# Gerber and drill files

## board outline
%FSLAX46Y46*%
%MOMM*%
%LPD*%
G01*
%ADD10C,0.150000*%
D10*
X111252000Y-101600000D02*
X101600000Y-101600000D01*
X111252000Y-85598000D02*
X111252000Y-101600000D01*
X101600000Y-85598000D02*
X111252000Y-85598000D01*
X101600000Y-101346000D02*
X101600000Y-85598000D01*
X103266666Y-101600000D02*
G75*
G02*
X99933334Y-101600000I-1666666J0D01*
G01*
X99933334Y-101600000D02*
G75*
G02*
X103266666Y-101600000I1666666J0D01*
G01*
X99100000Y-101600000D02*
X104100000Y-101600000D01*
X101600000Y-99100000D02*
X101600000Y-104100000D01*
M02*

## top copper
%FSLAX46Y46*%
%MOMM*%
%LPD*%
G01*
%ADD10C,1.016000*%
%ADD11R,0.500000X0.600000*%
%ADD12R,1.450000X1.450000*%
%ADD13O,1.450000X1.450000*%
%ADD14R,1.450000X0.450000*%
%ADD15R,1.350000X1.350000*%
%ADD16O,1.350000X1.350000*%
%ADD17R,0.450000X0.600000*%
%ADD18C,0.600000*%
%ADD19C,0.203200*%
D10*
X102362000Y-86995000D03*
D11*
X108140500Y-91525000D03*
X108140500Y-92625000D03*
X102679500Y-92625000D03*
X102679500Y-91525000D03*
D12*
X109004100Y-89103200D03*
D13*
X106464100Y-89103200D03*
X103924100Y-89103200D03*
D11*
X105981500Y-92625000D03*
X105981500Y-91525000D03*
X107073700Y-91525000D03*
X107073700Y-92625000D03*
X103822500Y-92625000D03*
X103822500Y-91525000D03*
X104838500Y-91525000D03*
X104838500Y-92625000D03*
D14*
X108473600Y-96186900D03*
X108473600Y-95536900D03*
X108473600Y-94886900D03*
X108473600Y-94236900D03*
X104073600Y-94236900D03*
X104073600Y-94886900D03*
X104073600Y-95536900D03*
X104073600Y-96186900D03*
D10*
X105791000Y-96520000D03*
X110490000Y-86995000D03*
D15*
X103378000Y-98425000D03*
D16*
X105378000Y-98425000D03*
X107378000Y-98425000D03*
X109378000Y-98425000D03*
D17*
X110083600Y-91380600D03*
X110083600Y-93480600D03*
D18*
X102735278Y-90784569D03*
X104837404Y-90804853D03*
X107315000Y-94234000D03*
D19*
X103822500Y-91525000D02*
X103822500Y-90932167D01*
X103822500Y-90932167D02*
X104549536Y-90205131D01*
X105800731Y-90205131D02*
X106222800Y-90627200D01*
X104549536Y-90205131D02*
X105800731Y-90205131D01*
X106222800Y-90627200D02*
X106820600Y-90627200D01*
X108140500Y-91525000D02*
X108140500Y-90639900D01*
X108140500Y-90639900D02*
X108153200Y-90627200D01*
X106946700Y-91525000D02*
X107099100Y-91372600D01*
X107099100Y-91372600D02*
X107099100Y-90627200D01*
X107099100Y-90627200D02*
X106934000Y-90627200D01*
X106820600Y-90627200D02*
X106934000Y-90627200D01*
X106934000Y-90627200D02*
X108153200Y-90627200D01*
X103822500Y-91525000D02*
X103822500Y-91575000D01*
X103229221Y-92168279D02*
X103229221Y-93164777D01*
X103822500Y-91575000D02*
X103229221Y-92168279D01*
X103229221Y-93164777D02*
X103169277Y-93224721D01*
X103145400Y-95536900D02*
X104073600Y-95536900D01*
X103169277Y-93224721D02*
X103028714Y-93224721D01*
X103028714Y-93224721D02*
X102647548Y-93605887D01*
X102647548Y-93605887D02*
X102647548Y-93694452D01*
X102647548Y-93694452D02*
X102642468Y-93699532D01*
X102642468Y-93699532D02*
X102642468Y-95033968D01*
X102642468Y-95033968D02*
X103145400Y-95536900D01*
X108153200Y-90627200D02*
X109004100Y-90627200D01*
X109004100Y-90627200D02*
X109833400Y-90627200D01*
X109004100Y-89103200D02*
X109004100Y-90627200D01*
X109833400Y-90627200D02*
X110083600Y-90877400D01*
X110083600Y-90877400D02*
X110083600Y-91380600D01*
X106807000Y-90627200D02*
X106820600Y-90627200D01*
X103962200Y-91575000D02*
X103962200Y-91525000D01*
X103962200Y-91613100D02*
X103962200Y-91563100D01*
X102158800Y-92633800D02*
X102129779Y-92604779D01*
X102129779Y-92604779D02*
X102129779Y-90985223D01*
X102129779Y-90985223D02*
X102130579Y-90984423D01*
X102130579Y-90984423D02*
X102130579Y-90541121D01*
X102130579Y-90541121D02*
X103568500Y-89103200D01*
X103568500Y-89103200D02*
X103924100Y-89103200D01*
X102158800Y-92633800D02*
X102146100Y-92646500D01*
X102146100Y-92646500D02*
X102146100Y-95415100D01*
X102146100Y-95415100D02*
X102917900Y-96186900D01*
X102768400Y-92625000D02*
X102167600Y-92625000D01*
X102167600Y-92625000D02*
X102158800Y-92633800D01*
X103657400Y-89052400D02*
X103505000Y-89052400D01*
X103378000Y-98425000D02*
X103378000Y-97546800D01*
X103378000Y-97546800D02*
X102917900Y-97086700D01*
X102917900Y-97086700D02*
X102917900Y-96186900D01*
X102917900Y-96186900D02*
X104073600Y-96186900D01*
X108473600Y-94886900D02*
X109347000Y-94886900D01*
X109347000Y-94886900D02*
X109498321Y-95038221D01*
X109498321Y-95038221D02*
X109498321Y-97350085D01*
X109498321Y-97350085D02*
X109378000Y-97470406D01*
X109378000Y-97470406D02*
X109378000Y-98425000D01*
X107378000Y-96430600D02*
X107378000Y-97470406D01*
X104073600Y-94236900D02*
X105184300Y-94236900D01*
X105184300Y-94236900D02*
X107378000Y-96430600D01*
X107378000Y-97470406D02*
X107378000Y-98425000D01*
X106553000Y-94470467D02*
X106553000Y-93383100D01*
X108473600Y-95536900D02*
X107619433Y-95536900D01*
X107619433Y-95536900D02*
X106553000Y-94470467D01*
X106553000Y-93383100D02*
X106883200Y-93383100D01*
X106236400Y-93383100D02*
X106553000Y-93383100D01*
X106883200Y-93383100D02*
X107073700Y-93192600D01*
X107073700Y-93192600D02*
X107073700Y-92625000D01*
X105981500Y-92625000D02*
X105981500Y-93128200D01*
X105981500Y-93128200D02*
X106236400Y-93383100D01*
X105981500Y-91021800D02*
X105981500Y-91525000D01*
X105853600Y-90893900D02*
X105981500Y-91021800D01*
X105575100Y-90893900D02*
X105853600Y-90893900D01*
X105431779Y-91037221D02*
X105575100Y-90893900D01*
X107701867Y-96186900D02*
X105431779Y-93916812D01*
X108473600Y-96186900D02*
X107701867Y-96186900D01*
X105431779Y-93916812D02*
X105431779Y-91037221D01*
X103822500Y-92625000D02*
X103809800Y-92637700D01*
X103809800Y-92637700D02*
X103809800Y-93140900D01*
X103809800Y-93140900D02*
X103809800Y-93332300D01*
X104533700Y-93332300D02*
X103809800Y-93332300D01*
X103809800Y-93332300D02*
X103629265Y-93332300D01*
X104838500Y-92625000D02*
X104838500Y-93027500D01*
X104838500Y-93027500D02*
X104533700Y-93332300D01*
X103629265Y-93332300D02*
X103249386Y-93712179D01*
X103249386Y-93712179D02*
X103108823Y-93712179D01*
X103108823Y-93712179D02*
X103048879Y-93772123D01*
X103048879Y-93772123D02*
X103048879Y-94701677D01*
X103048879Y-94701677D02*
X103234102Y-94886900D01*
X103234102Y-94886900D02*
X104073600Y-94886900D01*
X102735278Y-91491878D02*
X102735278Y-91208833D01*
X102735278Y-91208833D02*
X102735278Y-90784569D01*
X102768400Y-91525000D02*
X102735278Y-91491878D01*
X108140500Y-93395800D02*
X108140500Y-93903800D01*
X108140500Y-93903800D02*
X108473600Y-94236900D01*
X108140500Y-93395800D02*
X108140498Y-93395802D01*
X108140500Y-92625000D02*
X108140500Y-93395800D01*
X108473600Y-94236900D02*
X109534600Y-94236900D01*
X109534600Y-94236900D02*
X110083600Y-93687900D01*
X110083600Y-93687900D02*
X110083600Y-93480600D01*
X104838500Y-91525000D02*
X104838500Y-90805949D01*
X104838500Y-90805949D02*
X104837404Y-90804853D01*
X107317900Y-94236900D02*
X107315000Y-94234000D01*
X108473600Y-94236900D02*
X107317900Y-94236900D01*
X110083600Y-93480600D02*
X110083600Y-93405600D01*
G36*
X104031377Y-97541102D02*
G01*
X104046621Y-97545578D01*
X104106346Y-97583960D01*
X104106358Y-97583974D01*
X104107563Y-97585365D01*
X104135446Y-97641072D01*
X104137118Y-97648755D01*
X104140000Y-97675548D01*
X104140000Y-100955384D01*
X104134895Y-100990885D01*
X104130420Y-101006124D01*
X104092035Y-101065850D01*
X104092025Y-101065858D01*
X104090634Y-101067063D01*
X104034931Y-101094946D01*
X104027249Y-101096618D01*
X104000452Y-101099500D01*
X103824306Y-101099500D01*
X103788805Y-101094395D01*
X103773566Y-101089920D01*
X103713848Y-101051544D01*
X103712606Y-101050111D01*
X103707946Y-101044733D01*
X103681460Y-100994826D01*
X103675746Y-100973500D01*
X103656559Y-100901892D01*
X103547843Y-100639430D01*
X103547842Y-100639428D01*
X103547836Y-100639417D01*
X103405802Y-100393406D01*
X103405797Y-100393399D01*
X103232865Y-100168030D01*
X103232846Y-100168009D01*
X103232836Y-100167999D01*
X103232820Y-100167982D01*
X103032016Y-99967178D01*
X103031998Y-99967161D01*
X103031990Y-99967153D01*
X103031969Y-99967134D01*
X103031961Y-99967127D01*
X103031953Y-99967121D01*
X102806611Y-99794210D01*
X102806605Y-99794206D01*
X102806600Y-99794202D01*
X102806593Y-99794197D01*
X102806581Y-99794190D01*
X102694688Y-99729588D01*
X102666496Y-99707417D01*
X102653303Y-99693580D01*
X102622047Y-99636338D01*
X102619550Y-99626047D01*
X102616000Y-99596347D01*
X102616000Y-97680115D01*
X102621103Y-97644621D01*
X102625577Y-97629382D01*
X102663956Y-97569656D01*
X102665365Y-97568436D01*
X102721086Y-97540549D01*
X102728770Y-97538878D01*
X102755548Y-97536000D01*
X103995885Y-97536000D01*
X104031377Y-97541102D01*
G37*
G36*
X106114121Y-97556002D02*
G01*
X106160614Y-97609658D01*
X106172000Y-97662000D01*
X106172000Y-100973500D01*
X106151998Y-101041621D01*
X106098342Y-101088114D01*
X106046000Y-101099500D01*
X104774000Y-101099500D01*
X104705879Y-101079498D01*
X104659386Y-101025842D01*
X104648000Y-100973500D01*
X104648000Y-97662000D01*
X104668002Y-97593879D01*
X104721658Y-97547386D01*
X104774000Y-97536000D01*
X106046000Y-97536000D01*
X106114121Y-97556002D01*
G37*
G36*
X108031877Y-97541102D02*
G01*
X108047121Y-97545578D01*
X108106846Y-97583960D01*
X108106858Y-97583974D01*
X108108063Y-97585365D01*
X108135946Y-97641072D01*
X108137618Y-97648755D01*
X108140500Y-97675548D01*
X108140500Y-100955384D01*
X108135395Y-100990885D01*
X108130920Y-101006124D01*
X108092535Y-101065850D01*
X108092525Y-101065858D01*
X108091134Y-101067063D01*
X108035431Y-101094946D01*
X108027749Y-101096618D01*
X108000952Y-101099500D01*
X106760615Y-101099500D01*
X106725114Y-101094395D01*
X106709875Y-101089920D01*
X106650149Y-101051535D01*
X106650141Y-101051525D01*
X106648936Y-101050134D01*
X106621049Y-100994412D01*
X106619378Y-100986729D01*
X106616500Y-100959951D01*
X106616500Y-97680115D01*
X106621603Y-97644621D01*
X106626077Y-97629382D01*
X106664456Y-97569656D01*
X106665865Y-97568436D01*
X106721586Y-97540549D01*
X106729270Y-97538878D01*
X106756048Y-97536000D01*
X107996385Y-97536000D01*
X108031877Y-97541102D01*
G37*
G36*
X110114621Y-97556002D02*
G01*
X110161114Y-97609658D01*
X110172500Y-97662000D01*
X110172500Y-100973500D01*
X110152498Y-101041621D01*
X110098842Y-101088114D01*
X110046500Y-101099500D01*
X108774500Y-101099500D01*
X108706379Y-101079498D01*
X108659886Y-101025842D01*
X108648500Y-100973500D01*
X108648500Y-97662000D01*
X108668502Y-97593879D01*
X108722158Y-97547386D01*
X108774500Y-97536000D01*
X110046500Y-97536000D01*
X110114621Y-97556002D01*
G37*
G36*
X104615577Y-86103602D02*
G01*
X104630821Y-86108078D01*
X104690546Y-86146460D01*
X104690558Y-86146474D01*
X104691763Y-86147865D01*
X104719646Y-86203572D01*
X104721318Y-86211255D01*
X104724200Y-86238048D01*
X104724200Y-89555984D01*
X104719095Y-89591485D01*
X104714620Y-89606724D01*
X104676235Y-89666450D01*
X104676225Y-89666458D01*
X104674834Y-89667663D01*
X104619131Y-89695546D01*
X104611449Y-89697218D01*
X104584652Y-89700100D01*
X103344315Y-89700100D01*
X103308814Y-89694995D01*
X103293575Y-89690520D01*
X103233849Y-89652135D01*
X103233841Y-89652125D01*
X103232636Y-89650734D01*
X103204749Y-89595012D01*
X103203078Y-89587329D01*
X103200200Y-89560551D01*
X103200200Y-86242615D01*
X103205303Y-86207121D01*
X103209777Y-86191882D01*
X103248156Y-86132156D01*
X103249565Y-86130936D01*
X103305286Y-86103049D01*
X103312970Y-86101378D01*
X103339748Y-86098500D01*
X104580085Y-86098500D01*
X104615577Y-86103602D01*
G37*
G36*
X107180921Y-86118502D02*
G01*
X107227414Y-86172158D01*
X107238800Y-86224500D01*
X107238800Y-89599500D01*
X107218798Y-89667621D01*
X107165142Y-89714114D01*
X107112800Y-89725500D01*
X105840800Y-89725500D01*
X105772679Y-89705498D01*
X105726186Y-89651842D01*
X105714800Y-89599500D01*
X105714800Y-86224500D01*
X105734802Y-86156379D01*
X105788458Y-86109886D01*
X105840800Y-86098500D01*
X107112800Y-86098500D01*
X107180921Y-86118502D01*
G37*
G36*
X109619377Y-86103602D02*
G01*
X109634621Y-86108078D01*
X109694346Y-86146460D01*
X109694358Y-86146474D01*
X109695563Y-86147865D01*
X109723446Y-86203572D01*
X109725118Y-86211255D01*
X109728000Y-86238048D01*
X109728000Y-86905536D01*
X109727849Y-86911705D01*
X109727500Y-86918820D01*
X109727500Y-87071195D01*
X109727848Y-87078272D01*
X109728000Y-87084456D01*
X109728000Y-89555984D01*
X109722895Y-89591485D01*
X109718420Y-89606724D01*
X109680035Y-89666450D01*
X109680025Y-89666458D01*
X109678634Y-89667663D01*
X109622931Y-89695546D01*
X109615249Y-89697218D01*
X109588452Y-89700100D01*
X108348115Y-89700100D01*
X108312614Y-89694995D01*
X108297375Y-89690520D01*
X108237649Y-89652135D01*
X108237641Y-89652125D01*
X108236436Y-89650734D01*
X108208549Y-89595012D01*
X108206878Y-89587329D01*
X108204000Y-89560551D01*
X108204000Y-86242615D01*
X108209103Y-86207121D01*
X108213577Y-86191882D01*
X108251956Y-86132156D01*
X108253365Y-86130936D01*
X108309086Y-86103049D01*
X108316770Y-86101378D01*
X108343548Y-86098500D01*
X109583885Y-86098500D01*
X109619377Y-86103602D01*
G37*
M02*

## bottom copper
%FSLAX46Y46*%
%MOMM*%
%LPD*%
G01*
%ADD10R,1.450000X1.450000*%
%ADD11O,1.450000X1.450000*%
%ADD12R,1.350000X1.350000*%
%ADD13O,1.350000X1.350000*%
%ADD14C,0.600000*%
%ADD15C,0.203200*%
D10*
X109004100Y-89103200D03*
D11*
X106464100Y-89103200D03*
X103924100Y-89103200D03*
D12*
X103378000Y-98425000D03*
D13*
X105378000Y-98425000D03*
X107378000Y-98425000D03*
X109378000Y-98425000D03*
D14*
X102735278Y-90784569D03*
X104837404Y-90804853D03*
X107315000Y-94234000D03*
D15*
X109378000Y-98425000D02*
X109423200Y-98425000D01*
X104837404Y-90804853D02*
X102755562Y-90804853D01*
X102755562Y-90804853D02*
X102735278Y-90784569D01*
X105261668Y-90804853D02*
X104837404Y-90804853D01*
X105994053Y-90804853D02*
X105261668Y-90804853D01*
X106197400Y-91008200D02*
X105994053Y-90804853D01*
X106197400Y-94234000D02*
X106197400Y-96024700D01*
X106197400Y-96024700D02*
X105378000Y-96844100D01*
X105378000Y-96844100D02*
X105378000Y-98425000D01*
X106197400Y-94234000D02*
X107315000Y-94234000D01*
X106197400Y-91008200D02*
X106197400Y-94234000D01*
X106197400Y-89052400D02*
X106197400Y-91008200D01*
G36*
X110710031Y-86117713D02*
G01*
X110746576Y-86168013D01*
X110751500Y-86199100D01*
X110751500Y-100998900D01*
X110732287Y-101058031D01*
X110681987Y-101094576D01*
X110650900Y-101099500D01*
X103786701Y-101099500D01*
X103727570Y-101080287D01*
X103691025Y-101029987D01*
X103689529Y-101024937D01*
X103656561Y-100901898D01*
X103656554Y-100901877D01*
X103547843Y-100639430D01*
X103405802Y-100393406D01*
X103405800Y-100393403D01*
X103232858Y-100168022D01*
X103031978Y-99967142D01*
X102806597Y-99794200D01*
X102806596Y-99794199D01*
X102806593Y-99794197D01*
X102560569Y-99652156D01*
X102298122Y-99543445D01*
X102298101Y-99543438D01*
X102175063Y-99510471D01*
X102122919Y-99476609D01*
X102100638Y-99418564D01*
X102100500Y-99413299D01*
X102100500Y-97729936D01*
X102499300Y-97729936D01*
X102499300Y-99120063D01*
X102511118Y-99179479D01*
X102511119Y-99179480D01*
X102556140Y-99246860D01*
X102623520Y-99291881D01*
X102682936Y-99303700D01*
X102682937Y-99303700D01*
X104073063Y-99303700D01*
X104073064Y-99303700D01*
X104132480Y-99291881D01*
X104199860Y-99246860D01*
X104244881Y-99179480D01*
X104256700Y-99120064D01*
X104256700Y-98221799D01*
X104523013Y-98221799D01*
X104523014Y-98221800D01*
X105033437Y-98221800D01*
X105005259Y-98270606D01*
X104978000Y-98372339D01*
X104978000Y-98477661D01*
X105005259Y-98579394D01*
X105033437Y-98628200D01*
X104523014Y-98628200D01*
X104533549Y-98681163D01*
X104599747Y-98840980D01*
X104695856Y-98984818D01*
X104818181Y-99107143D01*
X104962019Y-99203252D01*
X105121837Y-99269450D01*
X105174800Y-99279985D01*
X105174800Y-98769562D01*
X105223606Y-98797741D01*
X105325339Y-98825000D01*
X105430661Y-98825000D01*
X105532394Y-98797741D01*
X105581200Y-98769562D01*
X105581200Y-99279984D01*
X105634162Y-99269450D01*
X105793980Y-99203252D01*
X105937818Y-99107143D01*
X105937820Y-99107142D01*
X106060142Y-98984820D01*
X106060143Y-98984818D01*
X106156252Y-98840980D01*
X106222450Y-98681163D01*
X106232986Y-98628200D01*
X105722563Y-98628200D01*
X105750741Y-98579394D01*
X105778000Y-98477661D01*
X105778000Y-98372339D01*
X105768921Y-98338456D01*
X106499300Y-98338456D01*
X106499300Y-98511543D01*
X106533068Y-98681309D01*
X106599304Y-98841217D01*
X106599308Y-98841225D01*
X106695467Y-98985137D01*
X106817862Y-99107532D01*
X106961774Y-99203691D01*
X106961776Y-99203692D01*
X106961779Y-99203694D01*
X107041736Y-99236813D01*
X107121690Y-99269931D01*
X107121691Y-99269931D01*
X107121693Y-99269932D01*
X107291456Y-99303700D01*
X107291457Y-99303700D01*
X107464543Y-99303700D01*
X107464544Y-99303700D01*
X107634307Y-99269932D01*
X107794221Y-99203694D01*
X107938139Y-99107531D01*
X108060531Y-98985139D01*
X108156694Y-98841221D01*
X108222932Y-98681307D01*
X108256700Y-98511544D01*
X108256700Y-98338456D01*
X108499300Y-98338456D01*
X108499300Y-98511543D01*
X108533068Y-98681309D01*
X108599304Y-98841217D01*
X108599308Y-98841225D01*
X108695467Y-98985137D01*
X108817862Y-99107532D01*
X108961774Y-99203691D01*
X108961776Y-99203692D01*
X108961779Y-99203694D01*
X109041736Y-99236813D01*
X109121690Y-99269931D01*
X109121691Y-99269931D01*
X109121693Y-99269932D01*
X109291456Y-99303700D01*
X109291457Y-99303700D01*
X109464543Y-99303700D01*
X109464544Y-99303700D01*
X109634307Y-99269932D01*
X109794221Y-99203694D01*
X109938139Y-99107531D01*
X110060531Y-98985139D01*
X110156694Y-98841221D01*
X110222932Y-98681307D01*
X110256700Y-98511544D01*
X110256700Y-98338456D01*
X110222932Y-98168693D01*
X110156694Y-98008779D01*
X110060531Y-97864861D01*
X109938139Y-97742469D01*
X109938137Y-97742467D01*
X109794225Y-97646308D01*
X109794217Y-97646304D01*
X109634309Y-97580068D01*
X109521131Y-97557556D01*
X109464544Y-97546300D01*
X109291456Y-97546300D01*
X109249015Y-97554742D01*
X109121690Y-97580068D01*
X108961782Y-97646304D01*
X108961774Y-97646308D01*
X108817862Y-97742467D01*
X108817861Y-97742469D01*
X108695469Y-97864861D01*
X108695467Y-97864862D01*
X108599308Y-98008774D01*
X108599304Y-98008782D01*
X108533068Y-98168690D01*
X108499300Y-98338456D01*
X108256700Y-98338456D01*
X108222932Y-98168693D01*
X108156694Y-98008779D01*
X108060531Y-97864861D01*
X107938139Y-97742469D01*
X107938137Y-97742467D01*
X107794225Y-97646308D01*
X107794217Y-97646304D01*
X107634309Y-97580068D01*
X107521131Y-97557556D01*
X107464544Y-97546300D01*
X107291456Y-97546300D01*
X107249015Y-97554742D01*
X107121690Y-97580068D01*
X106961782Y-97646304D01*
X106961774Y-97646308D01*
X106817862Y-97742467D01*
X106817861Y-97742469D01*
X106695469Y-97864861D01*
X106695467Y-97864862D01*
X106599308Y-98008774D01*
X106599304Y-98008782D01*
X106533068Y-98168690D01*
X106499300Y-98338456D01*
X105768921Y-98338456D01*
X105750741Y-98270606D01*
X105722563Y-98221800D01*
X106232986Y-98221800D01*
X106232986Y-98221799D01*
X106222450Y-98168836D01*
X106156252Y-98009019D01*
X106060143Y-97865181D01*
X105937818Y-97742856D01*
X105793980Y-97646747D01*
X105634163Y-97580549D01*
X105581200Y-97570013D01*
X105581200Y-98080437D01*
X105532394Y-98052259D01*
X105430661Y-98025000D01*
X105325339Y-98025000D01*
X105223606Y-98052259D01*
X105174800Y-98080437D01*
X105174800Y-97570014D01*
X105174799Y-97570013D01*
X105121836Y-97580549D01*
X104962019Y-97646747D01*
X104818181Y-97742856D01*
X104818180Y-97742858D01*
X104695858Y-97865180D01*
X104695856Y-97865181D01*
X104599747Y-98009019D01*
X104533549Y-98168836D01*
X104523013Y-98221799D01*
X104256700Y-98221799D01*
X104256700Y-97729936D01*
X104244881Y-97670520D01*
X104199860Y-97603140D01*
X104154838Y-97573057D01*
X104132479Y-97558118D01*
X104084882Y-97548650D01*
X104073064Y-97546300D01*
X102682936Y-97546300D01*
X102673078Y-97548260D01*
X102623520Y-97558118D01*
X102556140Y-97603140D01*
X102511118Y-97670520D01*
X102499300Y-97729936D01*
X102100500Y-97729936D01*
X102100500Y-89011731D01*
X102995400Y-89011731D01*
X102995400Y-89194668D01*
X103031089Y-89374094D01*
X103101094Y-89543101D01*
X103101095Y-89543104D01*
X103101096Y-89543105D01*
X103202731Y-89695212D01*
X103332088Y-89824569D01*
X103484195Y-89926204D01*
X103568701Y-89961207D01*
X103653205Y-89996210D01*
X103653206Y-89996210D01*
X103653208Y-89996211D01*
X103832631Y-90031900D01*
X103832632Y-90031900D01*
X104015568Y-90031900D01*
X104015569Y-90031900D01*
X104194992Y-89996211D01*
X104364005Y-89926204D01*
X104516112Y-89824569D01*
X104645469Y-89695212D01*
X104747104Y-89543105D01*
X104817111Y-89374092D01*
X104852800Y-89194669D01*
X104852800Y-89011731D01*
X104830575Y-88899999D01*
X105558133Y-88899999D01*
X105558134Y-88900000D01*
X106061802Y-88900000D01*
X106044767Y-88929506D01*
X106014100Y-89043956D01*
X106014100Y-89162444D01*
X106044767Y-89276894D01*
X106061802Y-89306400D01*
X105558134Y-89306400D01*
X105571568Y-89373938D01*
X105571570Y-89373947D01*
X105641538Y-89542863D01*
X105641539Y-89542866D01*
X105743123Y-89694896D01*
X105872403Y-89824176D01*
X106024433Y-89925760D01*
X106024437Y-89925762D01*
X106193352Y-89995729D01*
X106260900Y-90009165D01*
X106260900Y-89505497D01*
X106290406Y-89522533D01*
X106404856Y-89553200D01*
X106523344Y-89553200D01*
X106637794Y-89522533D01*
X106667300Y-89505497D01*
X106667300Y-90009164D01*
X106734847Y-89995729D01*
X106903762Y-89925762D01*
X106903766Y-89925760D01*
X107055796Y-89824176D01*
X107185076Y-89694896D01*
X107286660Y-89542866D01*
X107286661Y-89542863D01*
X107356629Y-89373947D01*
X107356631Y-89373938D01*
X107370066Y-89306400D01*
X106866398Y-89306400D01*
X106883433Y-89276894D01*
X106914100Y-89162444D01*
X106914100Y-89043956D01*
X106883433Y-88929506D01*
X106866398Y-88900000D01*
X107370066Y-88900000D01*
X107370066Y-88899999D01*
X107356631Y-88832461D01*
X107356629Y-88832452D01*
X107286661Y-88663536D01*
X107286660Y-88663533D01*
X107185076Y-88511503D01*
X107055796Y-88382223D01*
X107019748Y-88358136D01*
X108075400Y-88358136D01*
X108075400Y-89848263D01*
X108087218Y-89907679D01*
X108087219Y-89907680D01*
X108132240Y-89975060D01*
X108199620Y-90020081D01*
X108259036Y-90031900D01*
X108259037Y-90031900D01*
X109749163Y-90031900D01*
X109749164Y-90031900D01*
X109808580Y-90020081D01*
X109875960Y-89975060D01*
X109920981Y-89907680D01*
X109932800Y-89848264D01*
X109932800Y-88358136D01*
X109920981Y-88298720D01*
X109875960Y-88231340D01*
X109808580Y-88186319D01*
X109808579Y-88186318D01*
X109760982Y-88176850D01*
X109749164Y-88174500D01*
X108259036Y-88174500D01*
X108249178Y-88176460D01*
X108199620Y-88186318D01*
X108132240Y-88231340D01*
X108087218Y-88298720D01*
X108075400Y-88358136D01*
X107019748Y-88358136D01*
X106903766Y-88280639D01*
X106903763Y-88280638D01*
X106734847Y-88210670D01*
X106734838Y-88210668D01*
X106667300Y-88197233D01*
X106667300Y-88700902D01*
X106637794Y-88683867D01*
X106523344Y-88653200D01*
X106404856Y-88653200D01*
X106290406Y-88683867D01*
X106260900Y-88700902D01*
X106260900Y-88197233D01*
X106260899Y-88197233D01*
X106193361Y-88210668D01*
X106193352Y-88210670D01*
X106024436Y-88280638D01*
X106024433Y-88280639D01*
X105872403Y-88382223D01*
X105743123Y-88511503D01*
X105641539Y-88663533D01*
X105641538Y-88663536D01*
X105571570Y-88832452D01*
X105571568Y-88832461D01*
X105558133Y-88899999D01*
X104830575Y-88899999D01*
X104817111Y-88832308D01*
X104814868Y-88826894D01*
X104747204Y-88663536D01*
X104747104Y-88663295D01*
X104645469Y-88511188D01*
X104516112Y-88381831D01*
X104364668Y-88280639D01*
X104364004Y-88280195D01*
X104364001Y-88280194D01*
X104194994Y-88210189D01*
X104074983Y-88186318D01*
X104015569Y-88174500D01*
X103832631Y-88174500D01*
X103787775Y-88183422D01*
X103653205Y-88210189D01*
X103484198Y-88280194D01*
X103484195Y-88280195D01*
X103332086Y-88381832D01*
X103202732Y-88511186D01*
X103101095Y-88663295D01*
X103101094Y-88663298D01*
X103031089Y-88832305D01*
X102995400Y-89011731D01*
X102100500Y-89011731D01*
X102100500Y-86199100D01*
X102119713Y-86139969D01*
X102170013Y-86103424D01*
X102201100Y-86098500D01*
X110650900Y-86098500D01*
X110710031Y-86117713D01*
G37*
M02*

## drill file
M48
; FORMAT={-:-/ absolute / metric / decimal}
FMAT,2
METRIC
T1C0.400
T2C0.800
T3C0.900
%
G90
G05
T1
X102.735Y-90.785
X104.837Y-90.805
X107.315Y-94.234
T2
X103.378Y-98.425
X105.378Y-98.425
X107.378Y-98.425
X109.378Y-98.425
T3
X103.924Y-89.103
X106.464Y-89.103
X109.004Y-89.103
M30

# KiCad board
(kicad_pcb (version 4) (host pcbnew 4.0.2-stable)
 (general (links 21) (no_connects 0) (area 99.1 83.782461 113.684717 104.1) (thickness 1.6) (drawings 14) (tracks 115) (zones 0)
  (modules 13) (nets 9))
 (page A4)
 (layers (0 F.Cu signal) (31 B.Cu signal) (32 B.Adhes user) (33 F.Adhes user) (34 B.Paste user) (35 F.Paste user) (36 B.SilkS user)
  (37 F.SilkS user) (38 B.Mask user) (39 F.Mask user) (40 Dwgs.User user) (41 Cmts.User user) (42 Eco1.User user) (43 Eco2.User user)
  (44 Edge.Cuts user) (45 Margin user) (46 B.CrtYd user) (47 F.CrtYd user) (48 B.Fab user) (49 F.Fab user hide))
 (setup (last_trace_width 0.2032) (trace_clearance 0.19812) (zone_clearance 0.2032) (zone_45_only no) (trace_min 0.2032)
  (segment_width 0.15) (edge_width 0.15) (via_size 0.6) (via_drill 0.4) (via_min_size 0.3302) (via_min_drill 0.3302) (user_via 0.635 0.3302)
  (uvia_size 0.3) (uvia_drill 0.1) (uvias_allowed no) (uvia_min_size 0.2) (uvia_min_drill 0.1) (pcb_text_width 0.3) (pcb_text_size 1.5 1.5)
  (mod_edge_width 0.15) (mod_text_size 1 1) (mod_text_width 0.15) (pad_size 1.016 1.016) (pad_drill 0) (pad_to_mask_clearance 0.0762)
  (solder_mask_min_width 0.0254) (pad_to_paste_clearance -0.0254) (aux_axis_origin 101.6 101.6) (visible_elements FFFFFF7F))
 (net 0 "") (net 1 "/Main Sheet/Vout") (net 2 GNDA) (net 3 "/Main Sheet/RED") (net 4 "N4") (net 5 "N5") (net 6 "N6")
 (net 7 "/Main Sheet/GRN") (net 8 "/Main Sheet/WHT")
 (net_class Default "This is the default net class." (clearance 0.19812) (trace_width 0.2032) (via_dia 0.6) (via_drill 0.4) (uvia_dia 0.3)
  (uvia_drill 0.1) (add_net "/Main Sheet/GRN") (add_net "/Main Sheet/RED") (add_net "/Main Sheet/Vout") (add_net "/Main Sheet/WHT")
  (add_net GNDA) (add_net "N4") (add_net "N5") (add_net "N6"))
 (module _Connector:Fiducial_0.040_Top (layer F.Cu) (at 102.362 86.995)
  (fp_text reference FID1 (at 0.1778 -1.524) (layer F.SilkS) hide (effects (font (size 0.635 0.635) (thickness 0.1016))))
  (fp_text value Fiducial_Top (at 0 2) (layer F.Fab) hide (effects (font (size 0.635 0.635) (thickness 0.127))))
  (pad 1 smd circle (at 0 0) (size 1.016 1.016) (layers F.Cu F.Mask) (solder_mask_margin 0.508) (zone_connect 0) (thermal_width 2.032)))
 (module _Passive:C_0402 (layer F.Cu) (at 108.1405 92.075 270)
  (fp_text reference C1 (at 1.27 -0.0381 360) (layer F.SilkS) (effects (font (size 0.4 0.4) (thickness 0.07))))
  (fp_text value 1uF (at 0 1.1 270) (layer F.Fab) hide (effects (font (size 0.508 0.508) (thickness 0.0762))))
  (pad 1 smd rect (at -0.55 0 270) (size 0.6 0.5) (layers F.Cu F.Paste F.Mask) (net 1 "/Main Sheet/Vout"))
  (pad 2 smd rect (at 0.55 0 270) (size 0.6 0.5) (layers F.Cu F.Paste F.Mask) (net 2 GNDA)))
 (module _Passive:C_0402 (layer F.Cu) (at 102.6795 92.075 90)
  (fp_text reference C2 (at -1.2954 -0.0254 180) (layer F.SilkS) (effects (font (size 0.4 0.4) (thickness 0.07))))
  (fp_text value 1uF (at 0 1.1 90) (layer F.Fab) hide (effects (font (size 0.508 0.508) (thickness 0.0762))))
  (pad 1 smd rect (at -0.55 0 90) (size 0.6 0.5) (layers F.Cu F.Paste F.Mask) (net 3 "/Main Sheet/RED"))
  (pad 2 smd rect (at 0.55 0 90) (size 0.6 0.5) (layers F.Cu F.Paste F.Mask) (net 2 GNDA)))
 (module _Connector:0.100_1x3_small (layer F.Cu) (at 106.4641 89.1032 270)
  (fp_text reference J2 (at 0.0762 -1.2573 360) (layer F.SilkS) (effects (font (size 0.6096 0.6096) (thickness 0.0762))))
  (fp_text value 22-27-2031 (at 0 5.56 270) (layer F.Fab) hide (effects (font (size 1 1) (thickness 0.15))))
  (pad 1 thru_hole rect (at 0 -2.54 270) (size 1.45 1.45) (drill 0.9) (layers *.Cu *.Mask F.SilkS) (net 1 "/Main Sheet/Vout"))
  (pad 2 thru_hole oval (at 0 0 270) (size 1.45 1.45) (drill 0.9) (layers *.Cu *.Mask F.SilkS) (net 2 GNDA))
  (pad 3 thru_hole oval (at 0 2.54 270) (size 1.45 1.45) (drill 0.9) (layers *.Cu *.Mask F.SilkS) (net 3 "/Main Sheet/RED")))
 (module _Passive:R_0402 (layer F.Cu) (at 105.9815 92.075 90)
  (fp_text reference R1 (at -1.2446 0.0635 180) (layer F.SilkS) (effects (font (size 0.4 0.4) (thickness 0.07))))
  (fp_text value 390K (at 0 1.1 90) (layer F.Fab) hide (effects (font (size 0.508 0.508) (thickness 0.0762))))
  (pad 1 smd rect (at -0.55 0 90) (size 0.6 0.5) (layers F.Cu F.Paste F.Mask) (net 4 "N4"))
  (pad 2 smd rect (at 0.55 0 90) (size 0.6 0.5) (layers F.Cu F.Paste F.Mask) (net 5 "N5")))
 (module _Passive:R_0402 (layer F.Cu) (at 107.0737 92.075 270)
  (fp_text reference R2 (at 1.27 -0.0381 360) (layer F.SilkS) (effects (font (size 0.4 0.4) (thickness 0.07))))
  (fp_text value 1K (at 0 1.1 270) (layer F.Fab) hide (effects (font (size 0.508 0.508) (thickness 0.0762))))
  (pad 1 smd rect (at -0.55 0 270) (size 0.6 0.5) (layers F.Cu F.Paste F.Mask) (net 1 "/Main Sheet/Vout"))
  (pad 2 smd rect (at 0.55 0 270) (size 0.6 0.5) (layers F.Cu F.Paste F.Mask) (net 4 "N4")))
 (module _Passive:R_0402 (layer F.Cu) (at 103.8225 92.075 90)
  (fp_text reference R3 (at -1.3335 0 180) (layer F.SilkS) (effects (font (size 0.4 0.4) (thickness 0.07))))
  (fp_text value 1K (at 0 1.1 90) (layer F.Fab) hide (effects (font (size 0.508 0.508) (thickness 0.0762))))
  (pad 1 smd rect (at -0.55 0 90) (size 0.6 0.5) (layers F.Cu F.Paste F.Mask) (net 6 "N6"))
  (pad 2 smd rect (at 0.55 0 90) (size 0.6 0.5) (layers F.Cu F.Paste F.Mask) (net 1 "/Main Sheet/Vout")))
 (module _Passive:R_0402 (layer F.Cu) (at 104.8385 92.075 270)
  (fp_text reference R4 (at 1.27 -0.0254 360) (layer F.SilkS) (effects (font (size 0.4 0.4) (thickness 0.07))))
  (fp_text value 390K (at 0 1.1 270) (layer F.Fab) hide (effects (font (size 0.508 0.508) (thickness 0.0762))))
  (pad 1 smd rect (at -0.55 0 270) (size 0.6 0.5) (layers F.Cu F.Paste F.Mask) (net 2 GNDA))
  (pad 2 smd rect (at 0.55 0 270) (size 0.6 0.5) (layers F.Cu F.Paste F.Mask) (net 6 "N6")))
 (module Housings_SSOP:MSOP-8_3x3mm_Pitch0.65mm (layer F.Cu) (at 106.2736 95.2119 180)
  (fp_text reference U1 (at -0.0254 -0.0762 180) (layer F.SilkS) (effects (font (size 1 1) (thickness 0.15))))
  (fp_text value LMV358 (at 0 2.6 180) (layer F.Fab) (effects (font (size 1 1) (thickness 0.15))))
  (pad 1 smd rect (at -2.2 -0.975 180) (size 1.45 0.45) (layers F.Cu F.Paste F.Mask) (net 5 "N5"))
  (pad 2 smd rect (at -2.2 -0.325 180) (size 1.45 0.45) (layers F.Cu F.Paste F.Mask) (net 4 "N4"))
  (pad 3 smd rect (at -2.2 0.325 180) (size 1.45 0.45) (layers F.Cu F.Paste F.Mask) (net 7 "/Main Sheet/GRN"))
  (pad 4 smd rect (at -2.2 0.975 180) (size 1.45 0.45) (layers F.Cu F.Paste F.Mask) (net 2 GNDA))
  (pad 5 smd rect (at 2.2 0.975 180) (size 1.45 0.45) (layers F.Cu F.Paste F.Mask) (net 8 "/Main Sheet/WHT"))
  (pad 6 smd rect (at 2.2 0.325 180) (size 1.45 0.45) (layers F.Cu F.Paste F.Mask) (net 6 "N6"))
  (pad 7 smd rect (at 2.2 -0.325 180) (size 1.45 0.45) (layers F.Cu F.Paste F.Mask) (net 1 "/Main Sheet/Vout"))
  (pad 8 smd rect (at 2.2 -0.975 180) (size 1.45 0.45) (layers F.Cu F.Paste F.Mask) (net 3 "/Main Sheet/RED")))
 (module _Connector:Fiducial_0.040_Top (layer F.Cu) (at 105.791 96.52)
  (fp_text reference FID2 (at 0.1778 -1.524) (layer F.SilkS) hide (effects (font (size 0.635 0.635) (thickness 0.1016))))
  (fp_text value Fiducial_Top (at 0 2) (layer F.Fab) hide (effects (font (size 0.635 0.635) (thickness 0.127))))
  (pad 1 smd circle (at 0 0) (size 1.016 1.016) (layers F.Cu F.Mask) (solder_mask_margin 0.508) (zone_connect 0) (thermal_width 2.032)))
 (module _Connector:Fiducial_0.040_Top (layer F.Cu) (at 110.49 86.995)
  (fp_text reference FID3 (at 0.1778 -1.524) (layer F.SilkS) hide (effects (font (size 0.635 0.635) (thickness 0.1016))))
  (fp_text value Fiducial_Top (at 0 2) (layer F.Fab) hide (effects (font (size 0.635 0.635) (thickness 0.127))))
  (pad 1 smd circle (at 0 0) (size 1.016 1.016) (layers F.Cu F.Mask) (solder_mask_margin 0.508) (zone_connect 0) (thermal_width 2.032)))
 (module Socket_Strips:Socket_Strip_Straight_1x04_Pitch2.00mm (layer F.Cu) (at 103.378 98.425 90)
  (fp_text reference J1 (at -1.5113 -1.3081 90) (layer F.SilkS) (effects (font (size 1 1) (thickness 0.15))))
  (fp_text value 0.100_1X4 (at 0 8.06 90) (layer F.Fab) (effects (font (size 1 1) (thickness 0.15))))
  (pad 1 thru_hole rect (at 0 0 90) (size 1.35 1.35) (drill 0.8) (layers *.Cu *.Mask) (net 3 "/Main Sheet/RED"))
  (pad 2 thru_hole oval (at 0 2 90) (size 1.35 1.35) (drill 0.8) (layers *.Cu *.Mask) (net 2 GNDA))
  (pad 3 thru_hole oval (at 0 4 90) (size 1.35 1.35) (drill 0.8) (layers *.Cu *.Mask) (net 8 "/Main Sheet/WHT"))
  (pad 4 thru_hole oval (at 0 6 90) (size 1.35 1.35) (drill 0.8) (layers *.Cu *.Mask) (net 7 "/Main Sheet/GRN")))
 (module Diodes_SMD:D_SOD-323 (layer F.Cu) (at 110.0836 92.4306 270)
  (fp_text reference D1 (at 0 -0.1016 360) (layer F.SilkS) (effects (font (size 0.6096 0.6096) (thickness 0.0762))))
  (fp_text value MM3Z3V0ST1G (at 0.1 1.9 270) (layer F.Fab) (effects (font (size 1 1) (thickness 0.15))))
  (pad 1 smd rect (at -1.05 0 270) (size 0.6 0.45) (layers F.Cu F.Paste F.Mask) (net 1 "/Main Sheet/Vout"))
  (pad 2 smd rect (at 1.05 0 270) (size 0.6 0.45) (layers F.Cu F.Paste F.Mask) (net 2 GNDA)))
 (gr_line (start 111.252 101.6) (end 101.6 101.6) (layer Edge.Cuts) (width 0.15))
 (gr_line (start 111.252 85.598) (end 111.252 101.6) (layer Edge.Cuts) (width 0.15))
 (gr_line (start 101.6 85.598) (end 111.252 85.598) (layer Edge.Cuts) (width 0.15))
 (gr_line (start 101.6 101.346) (end 101.6 85.598) (layer Edge.Cuts) (width 0.15))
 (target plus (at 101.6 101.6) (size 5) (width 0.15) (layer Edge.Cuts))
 (segment (start 103.8225 91.525) (end 103.8225 90.932167) (width 0.2032) (layer F.Cu) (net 1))
 (segment (start 103.8225 90.932167) (end 104.549536 90.205131) (width 0.2032) (layer F.Cu) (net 1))
 (segment (start 105.800731 90.205131) (end 106.2228 90.6272) (width 0.2032) (layer F.Cu) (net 1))
 (segment (start 104.549536 90.205131) (end 105.800731 90.205131) (width 0.2032) (layer F.Cu) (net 1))
 (segment (start 106.2228 90.6272) (end 106.8206 90.6272) (width 0.2032) (layer F.Cu) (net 1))
 (segment (start 108.1405 91.525) (end 108.1405 90.6399) (width 0.2032) (layer F.Cu) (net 1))
 (segment (start 108.1405 90.6399) (end 108.1532 90.6272) (width 0.2032) (layer F.Cu) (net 1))
 (segment (start 106.9467 91.525) (end 107.0991 91.3726) (width 0.2032) (layer F.Cu) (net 1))
 (segment (start 107.0991 91.3726) (end 107.0991 90.6272) (width 0.2032) (layer F.Cu) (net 1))
 (segment (start 107.0991 90.6272) (end 106.934 90.6272) (width 0.2032) (layer F.Cu) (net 1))
 (segment (start 106.8206 90.6272) (end 106.934 90.6272) (width 0.2032) (layer F.Cu) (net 1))
 (segment (start 106.934 90.6272) (end 108.1532 90.6272) (width 0.2032) (layer F.Cu) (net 1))
 (segment (start 103.8225 91.525) (end 103.8225 91.575) (width 0.2032) (layer F.Cu) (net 1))
 (segment (start 103.229221 92.168279) (end 103.229221 93.164777) (width 0.2032) (layer F.Cu) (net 1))
 (segment (start 103.8225 91.575) (end 103.229221 92.168279) (width 0.2032) (layer F.Cu) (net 1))
 (segment (start 103.229221 93.164777) (end 103.169277 93.224721) (width 0.2032) (layer F.Cu) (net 1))
 (segment (start 103.1454 95.5369) (end 104.0736 95.5369) (width 0.2032) (layer F.Cu) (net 1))
 (segment (start 103.169277 93.224721) (end 103.028714 93.224721) (width 0.2032) (layer F.Cu) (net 1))
 (segment (start 103.028714 93.224721) (end 102.647548 93.605887) (width 0.2032) (layer F.Cu) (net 1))
 (segment (start 102.647548 93.605887) (end 102.647548 93.694452) (width 0.2032) (layer F.Cu) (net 1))
 (segment (start 102.647548 93.694452) (end 102.642468 93.699532) (width 0.2032) (layer F.Cu) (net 1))
 (segment (start 102.642468 93.699532) (end 102.642468 95.033968) (width 0.2032) (layer F.Cu) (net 1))
 (segment (start 102.642468 95.033968) (end 103.1454 95.5369) (width 0.2032) (layer F.Cu) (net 1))
 (segment (start 108.1532 90.6272) (end 109.0041 90.6272) (width 0.2032) (layer F.Cu) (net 1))
 (segment (start 109.0041 90.6272) (end 109.8334 90.6272) (width 0.2032) (layer F.Cu) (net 1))
 (segment (start 109.0041 89.1032) (end 109.0041 90.6272) (width 0.2032) (layer F.Cu) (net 1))
 (segment (start 109.8334 90.6272) (end 110.0836 90.8774) (width 0.2032) (layer F.Cu) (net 1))
 (segment (start 110.0836 90.8774) (end 110.0836 91.3806) (width 0.2032) (layer F.Cu) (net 1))
 (segment (start 106.807 90.6272) (end 106.8206 90.6272) (width 0.2032) (layer F.Cu) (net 1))
 (segment (start 103.9622 91.575) (end 103.9622 91.525) (width 0.2032) (layer F.Cu) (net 1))
 (segment (start 103.9622 91.6131) (end 103.9622 91.5631) (width 0.2032) (layer F.Cu) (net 1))
 (segment (start 102.1588 92.6338) (end 102.129779 92.604779) (width 0.2032) (layer F.Cu) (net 3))
 (segment (start 102.129779 92.604779) (end 102.129779 90.985223) (width 0.2032) (layer F.Cu) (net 3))
 (segment (start 102.129779 90.985223) (end 102.130579 90.984423) (width 0.2032) (layer F.Cu) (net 3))
 (segment (start 102.130579 90.984423) (end 102.130579 90.541121) (width 0.2032) (layer F.Cu) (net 3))
 (segment (start 102.130579 90.541121) (end 103.5685 89.1032) (width 0.2032) (layer F.Cu) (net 3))
 (segment (start 103.5685 89.1032) (end 103.9241 89.1032) (width 0.2032) (layer F.Cu) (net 3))
 (segment (start 102.1588 92.6338) (end 102.1461 92.6465) (width 0.2032) (layer F.Cu) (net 3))
 (segment (start 102.1461 92.6465) (end 102.1461 95.4151) (width 0.2032) (layer F.Cu) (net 3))
 (segment (start 102.1461 95.4151) (end 102.9179 96.1869) (width 0.2032) (layer F.Cu) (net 3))
 (segment (start 102.7684 92.625) (end 102.1676 92.625) (width 0.2032) (layer F.Cu) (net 3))
 (segment (start 102.1676 92.625) (end 102.1588 92.6338) (width 0.2032) (layer F.Cu) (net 3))
 (segment (start 103.6574 89.0524) (end 103.505 89.0524) (width 0.2032) (layer F.Cu) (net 3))
 (segment (start 103.378 98.425) (end 103.378 97.5468) (width 0.2032) (layer F.Cu) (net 3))
 (segment (start 103.378 97.5468) (end 102.9179 97.0867) (width 0.2032) (layer F.Cu) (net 3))
 (segment (start 102.9179 97.0867) (end 102.9179 96.1869) (width 0.2032) (layer F.Cu) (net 3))
 (segment (start 102.9179 96.1869) (end 104.0736 96.1869) (width 0.2032) (layer F.Cu) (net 3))
 (segment (start 108.4736 94.8869) (end 109.347 94.8869) (width 0.2032) (layer F.Cu) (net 7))
 (segment (start 109.347 94.8869) (end 109.498321 95.038221) (width 0.2032) (layer F.Cu) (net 7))
 (segment (start 109.498321 95.038221) (end 109.498321 97.350085) (width 0.2032) (layer F.Cu) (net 7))
 (segment (start 109.498321 97.350085) (end 109.378 97.470406) (width 0.2032) (layer F.Cu) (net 7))
 (segment (start 109.378 97.470406) (end 109.378 98.425) (width 0.2032) (layer F.Cu) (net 7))
 (segment (start 109.378 98.425) (end 109.4232 98.425) (width 0.2032) (layer B.Cu) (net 7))
 (segment (start 107.378 96.4306) (end 107.378 97.470406) (width 0.2032) (layer F.Cu) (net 8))
 (segment (start 104.0736 94.2369) (end 105.1843 94.2369) (width 0.2032) (layer F.Cu) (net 8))
 (segment (start 105.1843 94.2369) (end 107.378 96.4306) (width 0.2032) (layer F.Cu) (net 8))
 (segment (start 107.378 97.470406) (end 107.378 98.425) (width 0.2032) (layer F.Cu) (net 8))
 (segment (start 106.553 94.470467) (end 106.553 93.3831) (width 0.2032) (layer F.Cu) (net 4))
 (segment (start 108.4736 95.5369) (end 107.619433 95.5369) (width 0.2032) (layer F.Cu) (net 4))
 (segment (start 107.619433 95.5369) (end 106.553 94.470467) (width 0.2032) (layer F.Cu) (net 4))
 (segment (start 106.553 93.3831) (end 106.8832 93.3831) (width 0.2032) (layer F.Cu) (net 4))
 (segment (start 106.2364 93.3831) (end 106.553 93.3831) (width 0.2032) (layer F.Cu) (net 4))
 (segment (start 106.8832 93.3831) (end 107.0737 93.1926) (width 0.2032) (layer F.Cu) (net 4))
 (segment (start 107.0737 93.1926) (end 107.0737 92.625) (width 0.2032) (layer F.Cu) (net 4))
 (segment (start 105.9815 92.625) (end 105.9815 93.1282) (width 0.2032) (layer F.Cu) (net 4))
 (segment (start 105.9815 93.1282) (end 106.2364 93.3831) (width 0.2032) (layer F.Cu) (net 4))
 (segment (start 105.9815 91.0218) (end 105.9815 91.525) (width 0.2032) (layer F.Cu) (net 5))
 (segment (start 105.8536 90.8939) (end 105.9815 91.0218) (width 0.2032) (layer F.Cu) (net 5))
 (segment (start 105.5751 90.8939) (end 105.8536 90.8939) (width 0.2032) (layer F.Cu) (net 5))
 (segment (start 105.431779 91.037221) (end 105.5751 90.8939) (width 0.2032) (layer F.Cu) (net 5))
 (segment (start 107.701867 96.1869) (end 105.431779 93.916812) (width 0.2032) (layer F.Cu) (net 5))
 (segment (start 108.4736 96.1869) (end 107.701867 96.1869) (width 0.2032) (layer F.Cu) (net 5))
 (segment (start 105.431779 93.916812) (end 105.431779 91.037221) (width 0.2032) (layer F.Cu) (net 5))
 (segment (start 103.8225 92.625) (end 103.8098 92.6377) (width 0.2032) (layer F.Cu) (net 6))
 (segment (start 103.8098 92.6377) (end 103.8098 93.1409) (width 0.2032) (layer F.Cu) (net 6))
 (segment (start 103.8098 93.1409) (end 103.8098 93.3323) (width 0.2032) (layer F.Cu) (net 6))
 (segment (start 104.5337 93.3323) (end 103.8098 93.3323) (width 0.2032) (layer F.Cu) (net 6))
 (segment (start 103.8098 93.3323) (end 103.629265 93.3323) (width 0.2032) (layer F.Cu) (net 6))
 (segment (start 104.8385 92.625) (end 104.8385 93.0275) (width 0.2032) (layer F.Cu) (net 6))
 (segment (start 104.8385 93.0275) (end 104.5337 93.3323) (width 0.2032) (layer F.Cu) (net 6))
 (segment (start 103.629265 93.3323) (end 103.249386 93.712179) (width 0.2032) (layer F.Cu) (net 6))
 (segment (start 103.249386 93.712179) (end 103.108823 93.712179) (width 0.2032) (layer F.Cu) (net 6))
 (segment (start 103.108823 93.712179) (end 103.048879 93.772123) (width 0.2032) (layer F.Cu) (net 6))
 (segment (start 103.048879 93.772123) (end 103.048879 94.701677) (width 0.2032) (layer F.Cu) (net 6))
 (segment (start 103.048879 94.701677) (end 103.234102 94.8869) (width 0.2032) (layer F.Cu) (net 6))
 (segment (start 103.234102 94.8869) (end 104.0736 94.8869) (width 0.2032) (layer F.Cu) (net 6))
 (segment (start 102.735278 91.491878) (end 102.735278 91.208833) (width 0.2032) (layer F.Cu) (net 2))
 (segment (start 104.837404 90.804853) (end 102.755562 90.804853) (width 0.2032) (layer B.Cu) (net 2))
 (segment (start 102.735278 91.208833) (end 102.735278 90.784569) (width 0.2032) (layer F.Cu) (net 2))
 (segment (start 102.755562 90.804853) (end 102.735278 90.784569) (width 0.2032) (layer B.Cu) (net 2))
 (via (at 102.735278 90.784569) (size 0.6) (drill 0.4) (layers F.Cu B.Cu) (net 2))
 (segment (start 102.7684 91.525) (end 102.735278 91.491878) (width 0.2032) (layer F.Cu) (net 2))
 (segment (start 108.1405 93.3958) (end 108.1405 93.9038) (width 0.2032) (layer F.Cu) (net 2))
 (segment (start 108.1405 93.9038) (end 108.4736 94.2369) (width 0.2032) (layer F.Cu) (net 2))
 (segment (start 108.1405 93.3958) (end 108.140498 93.395802) (width 0.2032) (layer F.Cu) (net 2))
 (segment (start 108.1405 92.625) (end 108.1405 93.3958) (width 0.2032) (layer F.Cu) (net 2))
 (segment (start 108.4736 94.2369) (end 109.5346 94.2369) (width 0.2032) (layer F.Cu) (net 2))
 (segment (start 109.5346 94.2369) (end 110.0836 93.6879) (width 0.2032) (layer F.Cu) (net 2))
 (segment (start 110.0836 93.6879) (end 110.0836 93.4806) (width 0.2032) (layer F.Cu) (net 2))
 (segment (start 104.8385 91.525) (end 104.8385 90.805949) (width 0.2032) (layer F.Cu) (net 2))
 (segment (start 105.261668 90.804853) (end 104.837404 90.804853) (width 0.2032) (layer B.Cu) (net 2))
 (segment (start 104.8385 90.805949) (end 104.837404 90.804853) (width 0.2032) (layer F.Cu) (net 2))
 (segment (start 105.994053 90.804853) (end 105.261668 90.804853) (width 0.2032) (layer B.Cu) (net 2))
 (segment (start 106.1974 91.0082) (end 105.994053 90.804853) (width 0.2032) (layer B.Cu) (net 2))
 (via (at 104.837404 90.804853) (size 0.6) (drill 0.4) (layers F.Cu B.Cu) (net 2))
 (segment (start 106.1974 94.234) (end 106.1974 96.0247) (width 0.2032) (layer B.Cu) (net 2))
 (segment (start 106.1974 96.0247) (end 105.378 96.8441) (width 0.2032) (layer B.Cu) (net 2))
 (segment (start 105.378 96.8441) (end 105.378 98.425) (width 0.2032) (layer B.Cu) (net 2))
 (segment (start 106.1974 94.234) (end 107.315 94.234) (width 0.2032) (layer B.Cu) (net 2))
 (segment (start 107.3179 94.2369) (end 107.315 94.234) (width 0.2032) (layer F.Cu) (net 2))
 (segment (start 108.4736 94.2369) (end 107.3179 94.2369) (width 0.2032) (layer F.Cu) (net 2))
 (via (at 107.315 94.234) (size 0.6) (drill 0.4) (layers F.Cu B.Cu) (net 2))
 (segment (start 110.0836 93.4806) (end 110.0836 93.4056) (width 0.2032) (layer F.Cu) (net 2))
 (segment (start 106.1974 91.0082) (end 106.1974 94.234) (width 0.2032) (layer B.Cu) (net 2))
 (segment (start 106.1974 89.0524) (end 106.1974 91.0082) (width 0.2032) (layer B.Cu) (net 2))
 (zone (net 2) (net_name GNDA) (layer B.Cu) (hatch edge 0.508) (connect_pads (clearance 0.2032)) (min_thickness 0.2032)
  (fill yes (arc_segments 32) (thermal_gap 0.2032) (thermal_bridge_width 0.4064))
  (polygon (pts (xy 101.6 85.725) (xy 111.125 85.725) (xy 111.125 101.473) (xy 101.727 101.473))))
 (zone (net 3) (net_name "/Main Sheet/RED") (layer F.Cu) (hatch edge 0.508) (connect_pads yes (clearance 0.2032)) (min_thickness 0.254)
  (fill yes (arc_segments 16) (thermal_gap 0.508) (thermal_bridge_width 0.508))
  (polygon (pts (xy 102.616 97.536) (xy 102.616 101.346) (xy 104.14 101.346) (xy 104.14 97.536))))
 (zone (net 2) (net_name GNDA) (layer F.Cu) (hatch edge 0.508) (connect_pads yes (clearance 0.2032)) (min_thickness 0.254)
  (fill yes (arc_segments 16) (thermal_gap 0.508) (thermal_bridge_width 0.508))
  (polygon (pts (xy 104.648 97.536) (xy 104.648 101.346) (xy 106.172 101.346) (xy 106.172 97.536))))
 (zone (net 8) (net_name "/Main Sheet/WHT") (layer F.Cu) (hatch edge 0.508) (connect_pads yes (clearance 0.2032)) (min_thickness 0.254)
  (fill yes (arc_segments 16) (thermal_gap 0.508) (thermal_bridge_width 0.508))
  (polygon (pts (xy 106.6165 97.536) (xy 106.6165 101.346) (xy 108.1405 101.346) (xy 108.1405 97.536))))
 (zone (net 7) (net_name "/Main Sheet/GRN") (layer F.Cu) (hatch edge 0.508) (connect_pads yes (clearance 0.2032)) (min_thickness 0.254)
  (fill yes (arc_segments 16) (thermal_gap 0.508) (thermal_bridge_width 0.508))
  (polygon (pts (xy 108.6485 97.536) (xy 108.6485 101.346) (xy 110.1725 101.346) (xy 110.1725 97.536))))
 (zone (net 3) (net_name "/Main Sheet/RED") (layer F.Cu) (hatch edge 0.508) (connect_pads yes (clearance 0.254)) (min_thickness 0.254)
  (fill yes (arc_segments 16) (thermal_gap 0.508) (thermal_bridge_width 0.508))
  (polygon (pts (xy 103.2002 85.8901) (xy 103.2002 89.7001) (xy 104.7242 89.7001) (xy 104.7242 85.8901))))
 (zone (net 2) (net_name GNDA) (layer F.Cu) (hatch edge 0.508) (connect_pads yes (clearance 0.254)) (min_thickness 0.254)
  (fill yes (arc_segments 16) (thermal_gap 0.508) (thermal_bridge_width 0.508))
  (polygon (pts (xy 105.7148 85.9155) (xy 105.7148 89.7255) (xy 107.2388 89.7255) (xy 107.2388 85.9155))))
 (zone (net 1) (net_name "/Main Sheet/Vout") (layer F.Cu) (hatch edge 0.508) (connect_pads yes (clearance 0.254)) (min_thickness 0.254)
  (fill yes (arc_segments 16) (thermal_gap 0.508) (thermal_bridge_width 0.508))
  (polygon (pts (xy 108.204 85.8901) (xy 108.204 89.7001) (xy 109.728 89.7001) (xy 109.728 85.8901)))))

